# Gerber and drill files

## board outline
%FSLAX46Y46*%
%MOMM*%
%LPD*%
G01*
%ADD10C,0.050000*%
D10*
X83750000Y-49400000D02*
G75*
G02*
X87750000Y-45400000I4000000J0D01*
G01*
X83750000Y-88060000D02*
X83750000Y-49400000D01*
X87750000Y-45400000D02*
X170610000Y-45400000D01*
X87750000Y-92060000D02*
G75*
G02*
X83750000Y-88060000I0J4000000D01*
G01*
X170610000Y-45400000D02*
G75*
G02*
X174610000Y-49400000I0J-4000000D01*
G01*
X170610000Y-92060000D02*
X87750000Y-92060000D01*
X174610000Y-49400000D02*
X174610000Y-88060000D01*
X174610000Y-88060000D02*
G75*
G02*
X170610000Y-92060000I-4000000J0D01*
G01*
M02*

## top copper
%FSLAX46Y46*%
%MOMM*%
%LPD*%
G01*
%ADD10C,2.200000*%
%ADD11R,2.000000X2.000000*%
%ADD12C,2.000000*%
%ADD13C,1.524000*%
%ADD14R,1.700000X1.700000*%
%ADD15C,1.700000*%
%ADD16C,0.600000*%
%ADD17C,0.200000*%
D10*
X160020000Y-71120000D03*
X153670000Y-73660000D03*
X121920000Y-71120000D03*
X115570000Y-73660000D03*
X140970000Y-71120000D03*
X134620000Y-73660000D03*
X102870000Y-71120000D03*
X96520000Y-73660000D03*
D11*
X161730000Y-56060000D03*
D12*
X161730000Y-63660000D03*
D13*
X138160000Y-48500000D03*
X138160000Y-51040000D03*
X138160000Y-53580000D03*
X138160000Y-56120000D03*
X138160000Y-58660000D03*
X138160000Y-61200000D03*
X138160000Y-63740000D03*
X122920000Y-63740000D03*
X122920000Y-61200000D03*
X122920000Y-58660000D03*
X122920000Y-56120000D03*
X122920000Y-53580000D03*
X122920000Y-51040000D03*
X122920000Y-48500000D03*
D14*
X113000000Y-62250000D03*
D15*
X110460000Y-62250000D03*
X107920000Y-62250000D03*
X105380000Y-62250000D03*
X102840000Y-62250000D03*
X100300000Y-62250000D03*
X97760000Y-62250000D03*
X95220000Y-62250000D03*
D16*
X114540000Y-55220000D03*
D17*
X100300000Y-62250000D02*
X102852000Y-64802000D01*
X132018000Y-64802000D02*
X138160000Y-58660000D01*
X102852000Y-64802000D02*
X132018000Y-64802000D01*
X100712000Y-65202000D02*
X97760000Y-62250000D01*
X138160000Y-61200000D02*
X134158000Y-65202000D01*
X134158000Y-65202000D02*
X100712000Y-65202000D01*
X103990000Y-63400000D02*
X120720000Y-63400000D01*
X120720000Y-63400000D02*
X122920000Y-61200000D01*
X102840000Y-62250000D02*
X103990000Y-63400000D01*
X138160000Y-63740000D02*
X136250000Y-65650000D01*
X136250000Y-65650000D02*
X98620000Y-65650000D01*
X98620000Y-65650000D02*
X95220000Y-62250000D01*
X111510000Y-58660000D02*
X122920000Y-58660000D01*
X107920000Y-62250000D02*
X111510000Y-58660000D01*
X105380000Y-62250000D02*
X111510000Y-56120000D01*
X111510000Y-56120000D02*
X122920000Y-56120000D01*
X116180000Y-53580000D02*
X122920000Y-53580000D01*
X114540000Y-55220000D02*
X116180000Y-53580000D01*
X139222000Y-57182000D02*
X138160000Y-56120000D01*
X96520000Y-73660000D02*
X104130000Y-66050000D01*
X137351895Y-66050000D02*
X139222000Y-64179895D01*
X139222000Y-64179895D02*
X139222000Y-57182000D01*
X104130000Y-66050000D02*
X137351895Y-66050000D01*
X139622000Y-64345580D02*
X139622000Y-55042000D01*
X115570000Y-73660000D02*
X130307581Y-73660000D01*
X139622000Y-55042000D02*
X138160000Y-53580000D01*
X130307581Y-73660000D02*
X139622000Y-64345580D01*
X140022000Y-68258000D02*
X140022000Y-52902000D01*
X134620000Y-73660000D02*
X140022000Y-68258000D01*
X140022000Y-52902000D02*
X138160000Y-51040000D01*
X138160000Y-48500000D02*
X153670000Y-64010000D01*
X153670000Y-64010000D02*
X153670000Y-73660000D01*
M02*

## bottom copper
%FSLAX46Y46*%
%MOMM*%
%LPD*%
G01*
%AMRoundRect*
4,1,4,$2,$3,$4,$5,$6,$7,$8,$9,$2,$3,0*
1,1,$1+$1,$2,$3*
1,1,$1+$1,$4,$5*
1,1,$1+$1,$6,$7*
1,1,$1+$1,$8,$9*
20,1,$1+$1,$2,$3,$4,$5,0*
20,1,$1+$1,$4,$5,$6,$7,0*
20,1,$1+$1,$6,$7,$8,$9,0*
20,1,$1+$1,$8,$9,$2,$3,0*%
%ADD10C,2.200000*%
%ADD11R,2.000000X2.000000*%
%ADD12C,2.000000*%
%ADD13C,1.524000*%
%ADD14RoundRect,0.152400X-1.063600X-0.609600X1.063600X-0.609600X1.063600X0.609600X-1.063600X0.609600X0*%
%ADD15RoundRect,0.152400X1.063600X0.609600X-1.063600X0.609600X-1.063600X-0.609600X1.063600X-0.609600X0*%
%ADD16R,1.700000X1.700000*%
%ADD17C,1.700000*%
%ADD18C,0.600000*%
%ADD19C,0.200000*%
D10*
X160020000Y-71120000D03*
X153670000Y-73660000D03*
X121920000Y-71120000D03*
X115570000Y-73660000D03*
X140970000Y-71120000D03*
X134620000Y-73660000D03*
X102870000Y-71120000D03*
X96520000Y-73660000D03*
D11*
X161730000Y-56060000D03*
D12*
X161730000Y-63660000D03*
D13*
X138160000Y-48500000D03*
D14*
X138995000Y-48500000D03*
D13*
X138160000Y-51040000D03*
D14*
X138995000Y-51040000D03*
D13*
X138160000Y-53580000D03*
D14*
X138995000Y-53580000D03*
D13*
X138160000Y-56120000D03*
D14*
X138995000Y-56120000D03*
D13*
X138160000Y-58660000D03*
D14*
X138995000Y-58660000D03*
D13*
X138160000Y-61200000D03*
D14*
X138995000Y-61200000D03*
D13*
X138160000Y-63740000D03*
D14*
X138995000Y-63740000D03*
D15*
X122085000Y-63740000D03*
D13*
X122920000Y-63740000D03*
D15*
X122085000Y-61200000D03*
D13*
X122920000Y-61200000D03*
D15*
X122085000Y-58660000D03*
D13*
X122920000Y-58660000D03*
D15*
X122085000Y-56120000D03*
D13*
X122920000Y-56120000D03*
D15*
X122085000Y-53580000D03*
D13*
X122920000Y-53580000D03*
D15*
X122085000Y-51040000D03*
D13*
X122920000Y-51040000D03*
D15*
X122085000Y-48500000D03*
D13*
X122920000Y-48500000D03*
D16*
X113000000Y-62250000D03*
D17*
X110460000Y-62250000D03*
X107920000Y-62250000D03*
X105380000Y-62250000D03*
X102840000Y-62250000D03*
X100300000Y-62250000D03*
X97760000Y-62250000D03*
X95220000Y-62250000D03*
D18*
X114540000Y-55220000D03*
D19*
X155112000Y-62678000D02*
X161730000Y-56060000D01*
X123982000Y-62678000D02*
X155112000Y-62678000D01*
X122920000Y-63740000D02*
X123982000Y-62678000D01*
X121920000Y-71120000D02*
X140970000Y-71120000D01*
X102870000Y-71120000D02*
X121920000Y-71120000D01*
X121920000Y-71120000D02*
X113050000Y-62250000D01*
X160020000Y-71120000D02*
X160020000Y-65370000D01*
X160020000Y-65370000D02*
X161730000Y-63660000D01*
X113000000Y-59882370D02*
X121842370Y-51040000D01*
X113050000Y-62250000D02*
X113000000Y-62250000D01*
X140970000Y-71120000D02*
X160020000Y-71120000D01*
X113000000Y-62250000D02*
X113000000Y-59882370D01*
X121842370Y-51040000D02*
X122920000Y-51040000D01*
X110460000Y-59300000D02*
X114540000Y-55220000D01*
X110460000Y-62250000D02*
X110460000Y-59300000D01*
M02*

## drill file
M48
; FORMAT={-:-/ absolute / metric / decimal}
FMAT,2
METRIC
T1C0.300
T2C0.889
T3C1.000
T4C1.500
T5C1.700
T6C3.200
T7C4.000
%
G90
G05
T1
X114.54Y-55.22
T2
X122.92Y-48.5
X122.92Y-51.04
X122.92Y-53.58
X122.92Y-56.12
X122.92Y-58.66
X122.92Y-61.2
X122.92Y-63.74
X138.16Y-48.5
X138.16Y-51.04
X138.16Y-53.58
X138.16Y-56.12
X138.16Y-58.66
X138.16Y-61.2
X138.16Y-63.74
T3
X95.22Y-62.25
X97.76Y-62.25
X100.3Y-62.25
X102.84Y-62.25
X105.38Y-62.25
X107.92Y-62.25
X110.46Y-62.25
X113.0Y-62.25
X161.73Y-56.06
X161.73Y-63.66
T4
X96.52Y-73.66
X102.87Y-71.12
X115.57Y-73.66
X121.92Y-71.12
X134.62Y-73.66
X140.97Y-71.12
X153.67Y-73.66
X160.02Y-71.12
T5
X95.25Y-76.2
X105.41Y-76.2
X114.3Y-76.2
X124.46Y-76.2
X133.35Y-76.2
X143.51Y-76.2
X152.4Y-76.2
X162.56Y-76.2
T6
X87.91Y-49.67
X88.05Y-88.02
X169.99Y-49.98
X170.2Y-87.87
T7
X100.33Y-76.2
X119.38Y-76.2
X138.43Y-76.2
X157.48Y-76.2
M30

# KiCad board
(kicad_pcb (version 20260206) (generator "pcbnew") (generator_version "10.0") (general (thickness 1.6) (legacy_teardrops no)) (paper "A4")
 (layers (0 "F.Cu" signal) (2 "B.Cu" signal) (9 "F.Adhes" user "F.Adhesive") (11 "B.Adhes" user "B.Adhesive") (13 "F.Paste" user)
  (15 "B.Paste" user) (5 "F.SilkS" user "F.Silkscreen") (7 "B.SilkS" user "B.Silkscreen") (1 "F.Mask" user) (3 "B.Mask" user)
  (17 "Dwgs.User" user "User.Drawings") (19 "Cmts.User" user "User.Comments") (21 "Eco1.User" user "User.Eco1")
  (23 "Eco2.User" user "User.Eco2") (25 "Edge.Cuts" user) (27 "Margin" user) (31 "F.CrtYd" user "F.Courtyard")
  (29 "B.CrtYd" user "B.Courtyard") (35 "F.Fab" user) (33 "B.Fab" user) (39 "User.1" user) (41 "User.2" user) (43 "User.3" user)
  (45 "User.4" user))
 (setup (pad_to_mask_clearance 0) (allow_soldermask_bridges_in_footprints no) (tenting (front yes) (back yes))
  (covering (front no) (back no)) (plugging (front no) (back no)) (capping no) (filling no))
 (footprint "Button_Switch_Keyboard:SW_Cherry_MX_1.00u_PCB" (layer "F.Cu") (at 160.02 71.12)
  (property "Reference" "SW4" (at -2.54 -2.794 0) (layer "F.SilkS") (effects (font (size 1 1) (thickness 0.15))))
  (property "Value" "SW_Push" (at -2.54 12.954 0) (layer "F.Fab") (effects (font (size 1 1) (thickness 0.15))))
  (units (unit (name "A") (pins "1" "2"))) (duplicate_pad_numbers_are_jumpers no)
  (pad "" np_thru_hole circle (at -7.62 5.08) (size 1.7 1.7) (drill 1.7) (layers "*.Cu" "*.Mask"))
  (pad "" np_thru_hole circle (at -2.54 5.08) (size 4 4) (drill 4) (layers "*.Cu" "*.Mask"))
  (pad "" np_thru_hole circle (at 2.54 5.08) (size 1.7 1.7) (drill 1.7) (layers "*.Cu" "*.Mask"))
  (pad "1" thru_hole circle (at 0 0) (size 2.2 2.2) (drill 1.5) (layers "*.Cu" "*.Mask") (remove_unused_layers no) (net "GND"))
  (pad "2" thru_hole circle (at -6.35 2.54) (size 2.2 2.2) (drill 1.5) (layers "*.Cu" "*.Mask") (remove_unused_layers no)
   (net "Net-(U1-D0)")))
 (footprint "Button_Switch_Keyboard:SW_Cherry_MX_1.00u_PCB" (layer "F.Cu") (at 121.92 71.12)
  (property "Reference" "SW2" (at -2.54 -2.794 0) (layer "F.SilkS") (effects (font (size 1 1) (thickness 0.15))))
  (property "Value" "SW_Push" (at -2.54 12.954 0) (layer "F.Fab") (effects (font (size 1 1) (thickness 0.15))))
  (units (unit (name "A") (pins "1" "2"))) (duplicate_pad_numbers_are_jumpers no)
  (pad "" np_thru_hole circle (at -7.62 5.08) (size 1.7 1.7) (drill 1.7) (layers "*.Cu" "*.Mask"))
  (pad "" np_thru_hole circle (at -2.54 5.08) (size 4 4) (drill 4) (layers "*.Cu" "*.Mask"))
  (pad "" np_thru_hole circle (at 2.54 5.08) (size 1.7 1.7) (drill 1.7) (layers "*.Cu" "*.Mask"))
  (pad "1" thru_hole circle (at 0 0) (size 2.2 2.2) (drill 1.5) (layers "*.Cu" "*.Mask") (remove_unused_layers no) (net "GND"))
  (pad "2" thru_hole circle (at -6.35 2.54) (size 2.2 2.2) (drill 1.5) (layers "*.Cu" "*.Mask") (remove_unused_layers no)
   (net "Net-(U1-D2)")))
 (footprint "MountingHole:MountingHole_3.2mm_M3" (layer "F.Cu") (at 88.05 88.02)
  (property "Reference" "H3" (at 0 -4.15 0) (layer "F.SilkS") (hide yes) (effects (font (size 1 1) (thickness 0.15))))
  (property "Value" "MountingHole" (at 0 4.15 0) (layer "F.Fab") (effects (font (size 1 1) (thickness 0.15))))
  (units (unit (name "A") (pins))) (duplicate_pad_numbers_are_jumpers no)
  (pad "" np_thru_hole circle (at 0 0) (size 3.2 3.2) (drill 3.2) (layers "*.Cu" "*.Mask")))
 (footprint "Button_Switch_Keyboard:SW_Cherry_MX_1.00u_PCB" (layer "F.Cu") (at 140.97 71.12)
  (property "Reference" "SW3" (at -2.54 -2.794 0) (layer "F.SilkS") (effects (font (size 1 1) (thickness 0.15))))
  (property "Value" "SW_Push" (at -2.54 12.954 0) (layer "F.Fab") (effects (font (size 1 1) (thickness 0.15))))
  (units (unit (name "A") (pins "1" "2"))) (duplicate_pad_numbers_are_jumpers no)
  (pad "" np_thru_hole circle (at -7.62 5.08) (size 1.7 1.7) (drill 1.7) (layers "*.Cu" "*.Mask"))
  (pad "" np_thru_hole circle (at -2.54 5.08) (size 4 4) (drill 4) (layers "*.Cu" "*.Mask"))
  (pad "" np_thru_hole circle (at 2.54 5.08) (size 1.7 1.7) (drill 1.7) (layers "*.Cu" "*.Mask"))
  (pad "1" thru_hole circle (at 0 0) (size 2.2 2.2) (drill 1.5) (layers "*.Cu" "*.Mask") (remove_unused_layers no) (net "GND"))
  (pad "2" thru_hole circle (at -6.35 2.54) (size 2.2 2.2) (drill 1.5) (layers "*.Cu" "*.Mask") (remove_unused_layers no)
   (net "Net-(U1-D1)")))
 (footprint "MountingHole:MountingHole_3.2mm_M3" (layer "F.Cu") (at 169.99 49.98)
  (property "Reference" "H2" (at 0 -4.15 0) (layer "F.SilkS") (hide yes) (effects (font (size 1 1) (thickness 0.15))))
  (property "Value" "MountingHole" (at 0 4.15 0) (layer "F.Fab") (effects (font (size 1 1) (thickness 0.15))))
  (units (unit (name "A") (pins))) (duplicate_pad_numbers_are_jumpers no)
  (pad "" np_thru_hole circle (at 0 0) (size 3.2 3.2) (drill 3.2) (layers "*.Cu" "*.Mask")))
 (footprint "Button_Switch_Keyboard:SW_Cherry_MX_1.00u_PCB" (layer "F.Cu") (at 102.87 71.12)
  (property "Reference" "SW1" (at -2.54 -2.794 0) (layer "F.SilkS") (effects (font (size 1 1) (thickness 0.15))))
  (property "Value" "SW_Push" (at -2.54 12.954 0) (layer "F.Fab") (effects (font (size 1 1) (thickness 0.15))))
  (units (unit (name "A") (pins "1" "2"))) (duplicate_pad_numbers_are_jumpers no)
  (pad "" np_thru_hole circle (at -7.62 5.08) (size 1.7 1.7) (drill 1.7) (layers "*.Cu" "*.Mask"))
  (pad "" np_thru_hole circle (at -2.54 5.08) (size 4 4) (drill 4) (layers "*.Cu" "*.Mask"))
  (pad "" np_thru_hole circle (at 2.54 5.08) (size 1.7 1.7) (drill 1.7) (layers "*.Cu" "*.Mask"))
  (pad "1" thru_hole circle (at 0 0) (size 2.2 2.2) (drill 1.5) (layers "*.Cu" "*.Mask") (remove_unused_layers no) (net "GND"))
  (pad "2" thru_hole circle (at -6.35 2.54) (size 2.2 2.2) (drill 1.5) (layers "*.Cu" "*.Mask") (remove_unused_layers no)
   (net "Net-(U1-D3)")))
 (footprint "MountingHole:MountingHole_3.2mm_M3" (layer "F.Cu") (at 87.91 49.67)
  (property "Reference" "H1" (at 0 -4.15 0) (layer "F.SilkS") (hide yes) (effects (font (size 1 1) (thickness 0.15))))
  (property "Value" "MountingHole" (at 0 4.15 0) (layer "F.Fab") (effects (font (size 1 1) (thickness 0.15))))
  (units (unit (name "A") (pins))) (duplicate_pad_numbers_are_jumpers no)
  (pad "" np_thru_hole circle (at 0 0) (size 3.2 3.2) (drill 3.2) (layers "*.Cu" "*.Mask")))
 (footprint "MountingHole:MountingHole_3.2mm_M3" (layer "F.Cu") (at 170.2 87.87)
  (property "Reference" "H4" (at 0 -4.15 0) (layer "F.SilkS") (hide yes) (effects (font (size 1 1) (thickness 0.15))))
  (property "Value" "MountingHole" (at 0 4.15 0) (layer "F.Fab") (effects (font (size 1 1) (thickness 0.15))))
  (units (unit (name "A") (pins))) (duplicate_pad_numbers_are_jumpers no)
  (pad "" np_thru_hole circle (at 0 0) (size 3.2 3.2) (drill 3.2) (layers "*.Cu" "*.Mask")))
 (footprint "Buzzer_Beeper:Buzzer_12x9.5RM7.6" (layer "B.Cu") (at 161.73 56.06 -90)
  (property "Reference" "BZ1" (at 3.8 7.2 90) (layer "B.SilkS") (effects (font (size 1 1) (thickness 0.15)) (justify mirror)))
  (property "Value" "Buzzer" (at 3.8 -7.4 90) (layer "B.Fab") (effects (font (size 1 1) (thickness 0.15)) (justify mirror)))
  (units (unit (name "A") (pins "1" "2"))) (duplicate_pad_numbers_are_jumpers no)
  (pad "1" thru_hole rect (at 0 0 270) (size 2 2) (drill 1) (layers "*.Cu" "*.Mask") (remove_unused_layers no) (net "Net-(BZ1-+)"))
  (pad "2" thru_hole circle (at 7.6 0 270) (size 2 2) (drill 1) (layers "*.Cu" "*.Mask") (remove_unused_layers no) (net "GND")))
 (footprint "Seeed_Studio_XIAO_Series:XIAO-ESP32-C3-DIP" (layer "B.Cu") (at 130.54 56.12 90)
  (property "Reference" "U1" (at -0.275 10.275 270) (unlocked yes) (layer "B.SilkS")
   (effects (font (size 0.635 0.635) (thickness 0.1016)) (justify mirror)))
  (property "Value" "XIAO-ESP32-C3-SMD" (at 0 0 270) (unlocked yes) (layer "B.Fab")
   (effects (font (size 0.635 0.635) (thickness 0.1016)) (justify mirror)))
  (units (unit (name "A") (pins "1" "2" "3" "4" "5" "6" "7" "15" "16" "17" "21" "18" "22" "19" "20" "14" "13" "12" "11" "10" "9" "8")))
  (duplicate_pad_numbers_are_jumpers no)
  (pad "1" thru_hole circle (at 7.62 7.62) (size 1.524 1.524) (drill 0.889) (layers "*.Cu" "*.Mask") (remove_unused_layers no)
   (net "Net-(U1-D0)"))
  (pad "1" smd roundrect (at 7.62 8.455) (size 2.432 1.524) (layers "B.Cu" "B.Mask") (roundrect_rratio 0.1) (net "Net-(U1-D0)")
   (thermal_bridge_angle 45))
  (pad "2" thru_hole circle (at 5.08 7.62) (size 1.524 1.524) (drill 0.889) (layers "*.Cu" "*.Mask") (remove_unused_layers no)
   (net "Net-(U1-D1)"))
  (pad "2" smd roundrect (at 5.08 8.455) (size 2.432 1.524) (layers "B.Cu" "B.Mask") (roundrect_rratio 0.1) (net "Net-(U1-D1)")
   (thermal_bridge_angle 45))
  (pad "3" thru_hole circle (at 2.54 7.62) (size 1.524 1.524) (drill 0.889) (layers "*.Cu" "*.Mask") (remove_unused_layers no)
   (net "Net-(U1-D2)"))
  (pad "3" smd roundrect (at 2.54 8.455) (size 2.432 1.524) (layers "B.Cu" "B.Mask") (roundrect_rratio 0.1) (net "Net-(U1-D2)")
   (thermal_bridge_angle 45))
  (pad "4" thru_hole circle (at 0 7.62) (size 1.524 1.524) (drill 0.889) (layers "*.Cu" "*.Mask") (remove_unused_layers no)
   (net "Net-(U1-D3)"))
  (pad "4" smd roundrect (at 0 8.455) (size 2.432 1.524) (layers "B.Cu" "B.Mask") (roundrect_rratio 0.1) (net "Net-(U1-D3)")
   (thermal_bridge_angle 45))
  (pad "5" thru_hole circle (at -2.54 7.62) (size 1.524 1.524) (drill 0.889) (layers "*.Cu" "*.Mask") (remove_unused_layers no) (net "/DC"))
  (pad "5" smd roundrect (at -2.54 8.455) (size 2.432 1.524) (layers "B.Cu" "B.Mask") (roundrect_rratio 0.1) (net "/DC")
   (thermal_bridge_angle 45))
  (pad "6" thru_hole circle (at -5.08 7.62) (size 1.524 1.524) (drill 0.889) (layers "*.Cu" "*.Mask") (remove_unused_layers no) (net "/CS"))
  (pad "6" smd roundrect (at -5.08 8.455) (size 2.432 1.524) (layers "B.Cu" "B.Mask") (roundrect_rratio 0.1) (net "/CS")
   (thermal_bridge_angle 45))
  (pad "7" thru_hole circle (at -7.62 7.62) (size 1.524 1.524) (drill 0.889) (layers "*.Cu" "*.Mask") (remove_unused_layers no) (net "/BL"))
  (pad "7" smd roundrect (at -7.62 8.455) (size 2.432 1.524) (layers "B.Cu" "B.Mask") (roundrect_rratio 0.1) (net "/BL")
   (thermal_bridge_angle 45))
  (pad "8" smd roundrect (at -7.62 -8.455 180) (size 2.432 1.524) (layers "B.Cu" "B.Mask") (roundrect_rratio 0.1) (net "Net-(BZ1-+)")
   (thermal_bridge_angle 45))
  (pad "8" thru_hole circle (at -7.62 -7.62 180) (size 1.524 1.524) (drill 0.889) (layers "*.Cu" "*.Mask") (remove_unused_layers no)
   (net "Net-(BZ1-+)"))
  (pad "9" smd roundrect (at -5.08 -8.455 180) (size 2.432 1.524) (layers "B.Cu" "B.Mask") (roundrect_rratio 0.1) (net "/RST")
   (thermal_bridge_angle 45))
  (pad "9" thru_hole circle (at -5.08 -7.62 180) (size 1.524 1.524) (drill 0.889) (layers "*.Cu" "*.Mask") (remove_unused_layers no)
   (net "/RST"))
  (pad "10" smd roundrect (at -2.54 -8.455 180) (size 2.432 1.524) (layers "B.Cu" "B.Mask") (roundrect_rratio 0.1) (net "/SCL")
   (thermal_bridge_angle 45))
  (pad "10" thru_hole circle (at -2.54 -7.62 180) (size 1.524 1.524) (drill 0.889) (layers "*.Cu" "*.Mask") (remove_unused_layers no)
   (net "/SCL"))
  (pad "11" smd roundrect (at 0 -8.455 180) (size 2.432 1.524) (layers "B.Cu" "B.Mask") (roundrect_rratio 0.1) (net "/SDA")
   (thermal_bridge_angle 45))
  (pad "11" thru_hole circle (at 0 -7.62 180) (size 1.524 1.524) (drill 0.889) (layers "*.Cu" "*.Mask") (remove_unused_layers no)
   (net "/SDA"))
  (pad "12" smd roundrect (at 2.54 -8.455 180) (size 2.432 1.524) (layers "B.Cu" "B.Mask") (roundrect_rratio 0.1) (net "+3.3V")
   (thermal_bridge_angle 45))
  (pad "12" thru_hole circle (at 2.54 -7.62 180) (size 1.524 1.524) (drill 0.889) (layers "*.Cu" "*.Mask") (remove_unused_layers no)
   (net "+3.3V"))
  (pad "13" smd roundrect (at 5.08 -8.455 180) (size 2.432 1.524) (layers "B.Cu" "B.Mask") (roundrect_rratio 0.1) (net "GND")
   (thermal_bridge_angle 45))
  (pad "13" thru_hole circle (at 5.08 -7.62 180) (size 1.524 1.524) (drill 0.889) (layers "*.Cu" "*.Mask") (remove_unused_layers no)
   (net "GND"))
  (pad "14" smd roundrect (at 7.62 -8.455 180) (size 2.432 1.524) (layers "B.Cu" "B.Mask") (roundrect_rratio 0.1)
   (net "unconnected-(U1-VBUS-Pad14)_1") (thermal_bridge_angle 45))
  (pad "14" thru_hole circle (at 7.62 -7.62 180) (size 1.524 1.524) (drill 0.889) (layers "*.Cu" "*.Mask") (remove_unused_layers no)
   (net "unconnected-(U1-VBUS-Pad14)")))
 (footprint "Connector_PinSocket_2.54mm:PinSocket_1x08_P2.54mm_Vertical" (layer "B.Cu") (at 113 62.25 90)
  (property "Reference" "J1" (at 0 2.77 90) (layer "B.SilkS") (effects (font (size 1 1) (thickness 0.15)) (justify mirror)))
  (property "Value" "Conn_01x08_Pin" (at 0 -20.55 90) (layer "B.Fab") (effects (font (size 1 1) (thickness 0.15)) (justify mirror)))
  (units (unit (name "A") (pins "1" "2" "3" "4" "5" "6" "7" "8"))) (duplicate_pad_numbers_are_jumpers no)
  (pad "1" thru_hole rect (at 0 0 90) (size 1.7 1.7) (drill 1) (layers "*.Cu" "*.Mask") (remove_unused_layers no) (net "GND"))
  (pad "2" thru_hole circle (at 0 -2.54 90) (size 1.7 1.7) (drill 1) (layers "*.Cu" "*.Mask") (remove_unused_layers no) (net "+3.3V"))
  (pad "3" thru_hole circle (at 0 -5.08 90) (size 1.7 1.7) (drill 1) (layers "*.Cu" "*.Mask") (remove_unused_layers no) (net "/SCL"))
  (pad "4" thru_hole circle (at 0 -7.62 90) (size 1.7 1.7) (drill 1) (layers "*.Cu" "*.Mask") (remove_unused_layers no) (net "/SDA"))
  (pad "5" thru_hole circle (at 0 -10.16 90) (size 1.7 1.7) (drill 1) (layers "*.Cu" "*.Mask") (remove_unused_layers no) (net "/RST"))
  (pad "6" thru_hole circle (at 0 -12.7 90) (size 1.7 1.7) (drill 1) (layers "*.Cu" "*.Mask") (remove_unused_layers no) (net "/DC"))
  (pad "7" thru_hole circle (at 0 -15.24 90) (size 1.7 1.7) (drill 1) (layers "*.Cu" "*.Mask") (remove_unused_layers no) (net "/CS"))
  (pad "8" thru_hole circle (at 0 -17.78 90) (size 1.7 1.7) (drill 1) (layers "*.Cu" "*.Mask") (remove_unused_layers no) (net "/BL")))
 (gr_arc (start 83.75 49.4) (mid 84.921573 46.571573) (end 87.75 45.4) (stroke (width 0.05) (type default)) (layer "Edge.Cuts"))
 (gr_line (start 83.75 88.06) (end 83.75 49.4) (stroke (width 0.05) (type default)) (layer "Edge.Cuts"))
 (gr_line (start 87.75 45.4) (end 170.61 45.4) (stroke (width 0.05) (type default)) (layer "Edge.Cuts"))
 (gr_arc (start 87.75 92.06) (mid 84.921573 90.888427) (end 83.75 88.06) (stroke (width 0.05) (type default)) (layer "Edge.Cuts"))
 (gr_arc (start 170.61 45.4) (mid 173.438427 46.571573) (end 174.61 49.4) (stroke (width 0.05) (type default)) (layer "Edge.Cuts"))
 (gr_line (start 170.61 92.06) (end 87.75 92.06) (stroke (width 0.05) (type default)) (layer "Edge.Cuts"))
 (gr_line (start 174.61 49.4) (end 174.61 88.06) (stroke (width 0.05) (type default)) (layer "Edge.Cuts"))
 (gr_arc (start 174.61 88.06) (mid 173.438427 90.888427) (end 170.61 92.06) (stroke (width 0.05) (type default)) (layer "Edge.Cuts"))
 (segment (start 155.112 62.678) (end 161.73 56.06) (width 0.2) (layer "B.Cu") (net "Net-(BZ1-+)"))
 (segment (start 123.982 62.678) (end 155.112 62.678) (width 0.2) (layer "B.Cu") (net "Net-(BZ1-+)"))
 (segment (start 122.92 63.74) (end 123.982 62.678) (width 0.2) (layer "B.Cu") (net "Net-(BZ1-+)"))
 (segment (start 121.92 71.12) (end 140.97 71.12) (width 0.2) (layer "B.Cu") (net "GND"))
 (segment (start 102.87 71.12) (end 121.92 71.12) (width 0.2) (layer "B.Cu") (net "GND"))
 (segment (start 121.92 71.12) (end 113.05 62.25) (width 0.2) (layer "B.Cu") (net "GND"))
 (segment (start 160.02 71.12) (end 160.02 65.37) (width 0.2) (layer "B.Cu") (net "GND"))
 (segment (start 160.02 65.37) (end 161.73 63.66) (width 0.2) (layer "B.Cu") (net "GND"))
 (segment (start 113 59.88237) (end 121.84237 51.04) (width 0.2) (layer "B.Cu") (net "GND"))
 (segment (start 113.05 62.25) (end 113 62.25) (width 0.2) (layer "B.Cu") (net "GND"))
 (segment (start 140.97 71.12) (end 160.02 71.12) (width 0.2) (layer "B.Cu") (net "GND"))
 (segment (start 113 62.25) (end 113 59.88237) (width 0.2) (layer "B.Cu") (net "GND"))
 (segment (start 121.84237 51.04) (end 122.92 51.04) (width 0.2) (layer "B.Cu") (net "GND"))
 (segment (start 100.3 62.25) (end 102.852 64.802) (width 0.2) (layer "F.Cu") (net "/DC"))
 (segment (start 132.018 64.802) (end 138.16 58.66) (width 0.2) (layer "F.Cu") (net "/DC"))
 (segment (start 102.852 64.802) (end 132.018 64.802) (width 0.2) (layer "F.Cu") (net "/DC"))
 (segment (start 100.712 65.202) (end 97.76 62.25) (width 0.2) (layer "F.Cu") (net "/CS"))
 (segment (start 138.16 61.2) (end 134.158 65.202) (width 0.2) (layer "F.Cu") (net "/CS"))
 (segment (start 134.158 65.202) (end 100.712 65.202) (width 0.2) (layer "F.Cu") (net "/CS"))
 (segment (start 103.99 63.4) (end 120.72 63.4) (width 0.2) (layer "F.Cu") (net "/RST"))
 (segment (start 120.72 63.4) (end 122.92 61.2) (width 0.2) (layer "F.Cu") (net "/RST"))
 (segment (start 102.84 62.25) (end 103.99 63.4) (width 0.2) (layer "F.Cu") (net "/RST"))
 (segment (start 138.16 63.74) (end 136.25 65.65) (width 0.2) (layer "F.Cu") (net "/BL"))
 (segment (start 136.25 65.65) (end 98.62 65.65) (width 0.2) (layer "F.Cu") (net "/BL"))
 (segment (start 98.62 65.65) (end 95.22 62.25) (width 0.2) (layer "F.Cu") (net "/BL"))
 (segment (start 111.51 58.66) (end 122.92 58.66) (width 0.2) (layer "F.Cu") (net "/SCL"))
 (segment (start 107.92 62.25) (end 111.51 58.66) (width 0.2) (layer "F.Cu") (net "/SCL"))
 (segment (start 105.38 62.25) (end 111.51 56.12) (width 0.2) (layer "F.Cu") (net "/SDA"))
 (segment (start 111.51 56.12) (end 122.92 56.12) (width 0.2) (layer "F.Cu") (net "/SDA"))
 (segment (start 116.18 53.58) (end 122.92 53.58) (width 0.2) (layer "F.Cu") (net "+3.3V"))
 (segment (start 114.54 55.22) (end 116.18 53.58) (width 0.2) (layer "F.Cu") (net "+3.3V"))
 (via (at 114.54 55.22) (size 0.6) (drill 0.3) (layers "F.Cu" "B.Cu") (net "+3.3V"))
 (segment (start 110.46 59.3) (end 114.54 55.22) (width 0.2) (layer "B.Cu") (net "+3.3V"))
 (segment (start 110.46 62.25) (end 110.46 59.3) (width 0.2) (layer "B.Cu") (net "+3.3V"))
 (segment (start 139.222 57.182) (end 138.16 56.12) (width 0.2) (layer "F.Cu") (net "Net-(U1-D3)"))
 (segment (start 96.52 73.66) (end 104.13 66.05) (width 0.2) (layer "F.Cu") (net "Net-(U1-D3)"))
 (segment (start 137.351895 66.05) (end 139.222 64.179895) (width 0.2) (layer "F.Cu") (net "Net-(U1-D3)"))
 (segment (start 139.222 64.179895) (end 139.222 57.182) (width 0.2) (layer "F.Cu") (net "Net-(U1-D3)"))
 (segment (start 104.13 66.05) (end 137.351895 66.05) (width 0.2) (layer "F.Cu") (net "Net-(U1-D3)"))
 (segment (start 139.622 64.34558) (end 139.622 55.042) (width 0.2) (layer "F.Cu") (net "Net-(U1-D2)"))
 (segment (start 115.57 73.66) (end 130.307581 73.66) (width 0.2) (layer "F.Cu") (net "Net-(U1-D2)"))
 (segment (start 139.622 55.042) (end 138.16 53.58) (width 0.2) (layer "F.Cu") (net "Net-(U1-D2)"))
 (segment (start 130.307581 73.66) (end 139.622 64.34558) (width 0.2) (layer "F.Cu") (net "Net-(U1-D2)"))
 (segment (start 140.022 68.258) (end 140.022 52.902) (width 0.2) (layer "F.Cu") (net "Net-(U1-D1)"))
 (segment (start 134.62 73.66) (end 140.022 68.258) (width 0.2) (layer "F.Cu") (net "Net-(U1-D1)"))
 (segment (start 140.022 52.902) (end 138.16 51.04) (width 0.2) (layer "F.Cu") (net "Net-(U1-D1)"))
 (segment (start 138.16 48.5) (end 153.67 64.01) (width 0.2) (layer "F.Cu") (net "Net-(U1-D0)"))
 (segment (start 153.67 64.01) (end 153.67 73.66) (width 0.2) (layer "F.Cu") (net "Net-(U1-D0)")))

